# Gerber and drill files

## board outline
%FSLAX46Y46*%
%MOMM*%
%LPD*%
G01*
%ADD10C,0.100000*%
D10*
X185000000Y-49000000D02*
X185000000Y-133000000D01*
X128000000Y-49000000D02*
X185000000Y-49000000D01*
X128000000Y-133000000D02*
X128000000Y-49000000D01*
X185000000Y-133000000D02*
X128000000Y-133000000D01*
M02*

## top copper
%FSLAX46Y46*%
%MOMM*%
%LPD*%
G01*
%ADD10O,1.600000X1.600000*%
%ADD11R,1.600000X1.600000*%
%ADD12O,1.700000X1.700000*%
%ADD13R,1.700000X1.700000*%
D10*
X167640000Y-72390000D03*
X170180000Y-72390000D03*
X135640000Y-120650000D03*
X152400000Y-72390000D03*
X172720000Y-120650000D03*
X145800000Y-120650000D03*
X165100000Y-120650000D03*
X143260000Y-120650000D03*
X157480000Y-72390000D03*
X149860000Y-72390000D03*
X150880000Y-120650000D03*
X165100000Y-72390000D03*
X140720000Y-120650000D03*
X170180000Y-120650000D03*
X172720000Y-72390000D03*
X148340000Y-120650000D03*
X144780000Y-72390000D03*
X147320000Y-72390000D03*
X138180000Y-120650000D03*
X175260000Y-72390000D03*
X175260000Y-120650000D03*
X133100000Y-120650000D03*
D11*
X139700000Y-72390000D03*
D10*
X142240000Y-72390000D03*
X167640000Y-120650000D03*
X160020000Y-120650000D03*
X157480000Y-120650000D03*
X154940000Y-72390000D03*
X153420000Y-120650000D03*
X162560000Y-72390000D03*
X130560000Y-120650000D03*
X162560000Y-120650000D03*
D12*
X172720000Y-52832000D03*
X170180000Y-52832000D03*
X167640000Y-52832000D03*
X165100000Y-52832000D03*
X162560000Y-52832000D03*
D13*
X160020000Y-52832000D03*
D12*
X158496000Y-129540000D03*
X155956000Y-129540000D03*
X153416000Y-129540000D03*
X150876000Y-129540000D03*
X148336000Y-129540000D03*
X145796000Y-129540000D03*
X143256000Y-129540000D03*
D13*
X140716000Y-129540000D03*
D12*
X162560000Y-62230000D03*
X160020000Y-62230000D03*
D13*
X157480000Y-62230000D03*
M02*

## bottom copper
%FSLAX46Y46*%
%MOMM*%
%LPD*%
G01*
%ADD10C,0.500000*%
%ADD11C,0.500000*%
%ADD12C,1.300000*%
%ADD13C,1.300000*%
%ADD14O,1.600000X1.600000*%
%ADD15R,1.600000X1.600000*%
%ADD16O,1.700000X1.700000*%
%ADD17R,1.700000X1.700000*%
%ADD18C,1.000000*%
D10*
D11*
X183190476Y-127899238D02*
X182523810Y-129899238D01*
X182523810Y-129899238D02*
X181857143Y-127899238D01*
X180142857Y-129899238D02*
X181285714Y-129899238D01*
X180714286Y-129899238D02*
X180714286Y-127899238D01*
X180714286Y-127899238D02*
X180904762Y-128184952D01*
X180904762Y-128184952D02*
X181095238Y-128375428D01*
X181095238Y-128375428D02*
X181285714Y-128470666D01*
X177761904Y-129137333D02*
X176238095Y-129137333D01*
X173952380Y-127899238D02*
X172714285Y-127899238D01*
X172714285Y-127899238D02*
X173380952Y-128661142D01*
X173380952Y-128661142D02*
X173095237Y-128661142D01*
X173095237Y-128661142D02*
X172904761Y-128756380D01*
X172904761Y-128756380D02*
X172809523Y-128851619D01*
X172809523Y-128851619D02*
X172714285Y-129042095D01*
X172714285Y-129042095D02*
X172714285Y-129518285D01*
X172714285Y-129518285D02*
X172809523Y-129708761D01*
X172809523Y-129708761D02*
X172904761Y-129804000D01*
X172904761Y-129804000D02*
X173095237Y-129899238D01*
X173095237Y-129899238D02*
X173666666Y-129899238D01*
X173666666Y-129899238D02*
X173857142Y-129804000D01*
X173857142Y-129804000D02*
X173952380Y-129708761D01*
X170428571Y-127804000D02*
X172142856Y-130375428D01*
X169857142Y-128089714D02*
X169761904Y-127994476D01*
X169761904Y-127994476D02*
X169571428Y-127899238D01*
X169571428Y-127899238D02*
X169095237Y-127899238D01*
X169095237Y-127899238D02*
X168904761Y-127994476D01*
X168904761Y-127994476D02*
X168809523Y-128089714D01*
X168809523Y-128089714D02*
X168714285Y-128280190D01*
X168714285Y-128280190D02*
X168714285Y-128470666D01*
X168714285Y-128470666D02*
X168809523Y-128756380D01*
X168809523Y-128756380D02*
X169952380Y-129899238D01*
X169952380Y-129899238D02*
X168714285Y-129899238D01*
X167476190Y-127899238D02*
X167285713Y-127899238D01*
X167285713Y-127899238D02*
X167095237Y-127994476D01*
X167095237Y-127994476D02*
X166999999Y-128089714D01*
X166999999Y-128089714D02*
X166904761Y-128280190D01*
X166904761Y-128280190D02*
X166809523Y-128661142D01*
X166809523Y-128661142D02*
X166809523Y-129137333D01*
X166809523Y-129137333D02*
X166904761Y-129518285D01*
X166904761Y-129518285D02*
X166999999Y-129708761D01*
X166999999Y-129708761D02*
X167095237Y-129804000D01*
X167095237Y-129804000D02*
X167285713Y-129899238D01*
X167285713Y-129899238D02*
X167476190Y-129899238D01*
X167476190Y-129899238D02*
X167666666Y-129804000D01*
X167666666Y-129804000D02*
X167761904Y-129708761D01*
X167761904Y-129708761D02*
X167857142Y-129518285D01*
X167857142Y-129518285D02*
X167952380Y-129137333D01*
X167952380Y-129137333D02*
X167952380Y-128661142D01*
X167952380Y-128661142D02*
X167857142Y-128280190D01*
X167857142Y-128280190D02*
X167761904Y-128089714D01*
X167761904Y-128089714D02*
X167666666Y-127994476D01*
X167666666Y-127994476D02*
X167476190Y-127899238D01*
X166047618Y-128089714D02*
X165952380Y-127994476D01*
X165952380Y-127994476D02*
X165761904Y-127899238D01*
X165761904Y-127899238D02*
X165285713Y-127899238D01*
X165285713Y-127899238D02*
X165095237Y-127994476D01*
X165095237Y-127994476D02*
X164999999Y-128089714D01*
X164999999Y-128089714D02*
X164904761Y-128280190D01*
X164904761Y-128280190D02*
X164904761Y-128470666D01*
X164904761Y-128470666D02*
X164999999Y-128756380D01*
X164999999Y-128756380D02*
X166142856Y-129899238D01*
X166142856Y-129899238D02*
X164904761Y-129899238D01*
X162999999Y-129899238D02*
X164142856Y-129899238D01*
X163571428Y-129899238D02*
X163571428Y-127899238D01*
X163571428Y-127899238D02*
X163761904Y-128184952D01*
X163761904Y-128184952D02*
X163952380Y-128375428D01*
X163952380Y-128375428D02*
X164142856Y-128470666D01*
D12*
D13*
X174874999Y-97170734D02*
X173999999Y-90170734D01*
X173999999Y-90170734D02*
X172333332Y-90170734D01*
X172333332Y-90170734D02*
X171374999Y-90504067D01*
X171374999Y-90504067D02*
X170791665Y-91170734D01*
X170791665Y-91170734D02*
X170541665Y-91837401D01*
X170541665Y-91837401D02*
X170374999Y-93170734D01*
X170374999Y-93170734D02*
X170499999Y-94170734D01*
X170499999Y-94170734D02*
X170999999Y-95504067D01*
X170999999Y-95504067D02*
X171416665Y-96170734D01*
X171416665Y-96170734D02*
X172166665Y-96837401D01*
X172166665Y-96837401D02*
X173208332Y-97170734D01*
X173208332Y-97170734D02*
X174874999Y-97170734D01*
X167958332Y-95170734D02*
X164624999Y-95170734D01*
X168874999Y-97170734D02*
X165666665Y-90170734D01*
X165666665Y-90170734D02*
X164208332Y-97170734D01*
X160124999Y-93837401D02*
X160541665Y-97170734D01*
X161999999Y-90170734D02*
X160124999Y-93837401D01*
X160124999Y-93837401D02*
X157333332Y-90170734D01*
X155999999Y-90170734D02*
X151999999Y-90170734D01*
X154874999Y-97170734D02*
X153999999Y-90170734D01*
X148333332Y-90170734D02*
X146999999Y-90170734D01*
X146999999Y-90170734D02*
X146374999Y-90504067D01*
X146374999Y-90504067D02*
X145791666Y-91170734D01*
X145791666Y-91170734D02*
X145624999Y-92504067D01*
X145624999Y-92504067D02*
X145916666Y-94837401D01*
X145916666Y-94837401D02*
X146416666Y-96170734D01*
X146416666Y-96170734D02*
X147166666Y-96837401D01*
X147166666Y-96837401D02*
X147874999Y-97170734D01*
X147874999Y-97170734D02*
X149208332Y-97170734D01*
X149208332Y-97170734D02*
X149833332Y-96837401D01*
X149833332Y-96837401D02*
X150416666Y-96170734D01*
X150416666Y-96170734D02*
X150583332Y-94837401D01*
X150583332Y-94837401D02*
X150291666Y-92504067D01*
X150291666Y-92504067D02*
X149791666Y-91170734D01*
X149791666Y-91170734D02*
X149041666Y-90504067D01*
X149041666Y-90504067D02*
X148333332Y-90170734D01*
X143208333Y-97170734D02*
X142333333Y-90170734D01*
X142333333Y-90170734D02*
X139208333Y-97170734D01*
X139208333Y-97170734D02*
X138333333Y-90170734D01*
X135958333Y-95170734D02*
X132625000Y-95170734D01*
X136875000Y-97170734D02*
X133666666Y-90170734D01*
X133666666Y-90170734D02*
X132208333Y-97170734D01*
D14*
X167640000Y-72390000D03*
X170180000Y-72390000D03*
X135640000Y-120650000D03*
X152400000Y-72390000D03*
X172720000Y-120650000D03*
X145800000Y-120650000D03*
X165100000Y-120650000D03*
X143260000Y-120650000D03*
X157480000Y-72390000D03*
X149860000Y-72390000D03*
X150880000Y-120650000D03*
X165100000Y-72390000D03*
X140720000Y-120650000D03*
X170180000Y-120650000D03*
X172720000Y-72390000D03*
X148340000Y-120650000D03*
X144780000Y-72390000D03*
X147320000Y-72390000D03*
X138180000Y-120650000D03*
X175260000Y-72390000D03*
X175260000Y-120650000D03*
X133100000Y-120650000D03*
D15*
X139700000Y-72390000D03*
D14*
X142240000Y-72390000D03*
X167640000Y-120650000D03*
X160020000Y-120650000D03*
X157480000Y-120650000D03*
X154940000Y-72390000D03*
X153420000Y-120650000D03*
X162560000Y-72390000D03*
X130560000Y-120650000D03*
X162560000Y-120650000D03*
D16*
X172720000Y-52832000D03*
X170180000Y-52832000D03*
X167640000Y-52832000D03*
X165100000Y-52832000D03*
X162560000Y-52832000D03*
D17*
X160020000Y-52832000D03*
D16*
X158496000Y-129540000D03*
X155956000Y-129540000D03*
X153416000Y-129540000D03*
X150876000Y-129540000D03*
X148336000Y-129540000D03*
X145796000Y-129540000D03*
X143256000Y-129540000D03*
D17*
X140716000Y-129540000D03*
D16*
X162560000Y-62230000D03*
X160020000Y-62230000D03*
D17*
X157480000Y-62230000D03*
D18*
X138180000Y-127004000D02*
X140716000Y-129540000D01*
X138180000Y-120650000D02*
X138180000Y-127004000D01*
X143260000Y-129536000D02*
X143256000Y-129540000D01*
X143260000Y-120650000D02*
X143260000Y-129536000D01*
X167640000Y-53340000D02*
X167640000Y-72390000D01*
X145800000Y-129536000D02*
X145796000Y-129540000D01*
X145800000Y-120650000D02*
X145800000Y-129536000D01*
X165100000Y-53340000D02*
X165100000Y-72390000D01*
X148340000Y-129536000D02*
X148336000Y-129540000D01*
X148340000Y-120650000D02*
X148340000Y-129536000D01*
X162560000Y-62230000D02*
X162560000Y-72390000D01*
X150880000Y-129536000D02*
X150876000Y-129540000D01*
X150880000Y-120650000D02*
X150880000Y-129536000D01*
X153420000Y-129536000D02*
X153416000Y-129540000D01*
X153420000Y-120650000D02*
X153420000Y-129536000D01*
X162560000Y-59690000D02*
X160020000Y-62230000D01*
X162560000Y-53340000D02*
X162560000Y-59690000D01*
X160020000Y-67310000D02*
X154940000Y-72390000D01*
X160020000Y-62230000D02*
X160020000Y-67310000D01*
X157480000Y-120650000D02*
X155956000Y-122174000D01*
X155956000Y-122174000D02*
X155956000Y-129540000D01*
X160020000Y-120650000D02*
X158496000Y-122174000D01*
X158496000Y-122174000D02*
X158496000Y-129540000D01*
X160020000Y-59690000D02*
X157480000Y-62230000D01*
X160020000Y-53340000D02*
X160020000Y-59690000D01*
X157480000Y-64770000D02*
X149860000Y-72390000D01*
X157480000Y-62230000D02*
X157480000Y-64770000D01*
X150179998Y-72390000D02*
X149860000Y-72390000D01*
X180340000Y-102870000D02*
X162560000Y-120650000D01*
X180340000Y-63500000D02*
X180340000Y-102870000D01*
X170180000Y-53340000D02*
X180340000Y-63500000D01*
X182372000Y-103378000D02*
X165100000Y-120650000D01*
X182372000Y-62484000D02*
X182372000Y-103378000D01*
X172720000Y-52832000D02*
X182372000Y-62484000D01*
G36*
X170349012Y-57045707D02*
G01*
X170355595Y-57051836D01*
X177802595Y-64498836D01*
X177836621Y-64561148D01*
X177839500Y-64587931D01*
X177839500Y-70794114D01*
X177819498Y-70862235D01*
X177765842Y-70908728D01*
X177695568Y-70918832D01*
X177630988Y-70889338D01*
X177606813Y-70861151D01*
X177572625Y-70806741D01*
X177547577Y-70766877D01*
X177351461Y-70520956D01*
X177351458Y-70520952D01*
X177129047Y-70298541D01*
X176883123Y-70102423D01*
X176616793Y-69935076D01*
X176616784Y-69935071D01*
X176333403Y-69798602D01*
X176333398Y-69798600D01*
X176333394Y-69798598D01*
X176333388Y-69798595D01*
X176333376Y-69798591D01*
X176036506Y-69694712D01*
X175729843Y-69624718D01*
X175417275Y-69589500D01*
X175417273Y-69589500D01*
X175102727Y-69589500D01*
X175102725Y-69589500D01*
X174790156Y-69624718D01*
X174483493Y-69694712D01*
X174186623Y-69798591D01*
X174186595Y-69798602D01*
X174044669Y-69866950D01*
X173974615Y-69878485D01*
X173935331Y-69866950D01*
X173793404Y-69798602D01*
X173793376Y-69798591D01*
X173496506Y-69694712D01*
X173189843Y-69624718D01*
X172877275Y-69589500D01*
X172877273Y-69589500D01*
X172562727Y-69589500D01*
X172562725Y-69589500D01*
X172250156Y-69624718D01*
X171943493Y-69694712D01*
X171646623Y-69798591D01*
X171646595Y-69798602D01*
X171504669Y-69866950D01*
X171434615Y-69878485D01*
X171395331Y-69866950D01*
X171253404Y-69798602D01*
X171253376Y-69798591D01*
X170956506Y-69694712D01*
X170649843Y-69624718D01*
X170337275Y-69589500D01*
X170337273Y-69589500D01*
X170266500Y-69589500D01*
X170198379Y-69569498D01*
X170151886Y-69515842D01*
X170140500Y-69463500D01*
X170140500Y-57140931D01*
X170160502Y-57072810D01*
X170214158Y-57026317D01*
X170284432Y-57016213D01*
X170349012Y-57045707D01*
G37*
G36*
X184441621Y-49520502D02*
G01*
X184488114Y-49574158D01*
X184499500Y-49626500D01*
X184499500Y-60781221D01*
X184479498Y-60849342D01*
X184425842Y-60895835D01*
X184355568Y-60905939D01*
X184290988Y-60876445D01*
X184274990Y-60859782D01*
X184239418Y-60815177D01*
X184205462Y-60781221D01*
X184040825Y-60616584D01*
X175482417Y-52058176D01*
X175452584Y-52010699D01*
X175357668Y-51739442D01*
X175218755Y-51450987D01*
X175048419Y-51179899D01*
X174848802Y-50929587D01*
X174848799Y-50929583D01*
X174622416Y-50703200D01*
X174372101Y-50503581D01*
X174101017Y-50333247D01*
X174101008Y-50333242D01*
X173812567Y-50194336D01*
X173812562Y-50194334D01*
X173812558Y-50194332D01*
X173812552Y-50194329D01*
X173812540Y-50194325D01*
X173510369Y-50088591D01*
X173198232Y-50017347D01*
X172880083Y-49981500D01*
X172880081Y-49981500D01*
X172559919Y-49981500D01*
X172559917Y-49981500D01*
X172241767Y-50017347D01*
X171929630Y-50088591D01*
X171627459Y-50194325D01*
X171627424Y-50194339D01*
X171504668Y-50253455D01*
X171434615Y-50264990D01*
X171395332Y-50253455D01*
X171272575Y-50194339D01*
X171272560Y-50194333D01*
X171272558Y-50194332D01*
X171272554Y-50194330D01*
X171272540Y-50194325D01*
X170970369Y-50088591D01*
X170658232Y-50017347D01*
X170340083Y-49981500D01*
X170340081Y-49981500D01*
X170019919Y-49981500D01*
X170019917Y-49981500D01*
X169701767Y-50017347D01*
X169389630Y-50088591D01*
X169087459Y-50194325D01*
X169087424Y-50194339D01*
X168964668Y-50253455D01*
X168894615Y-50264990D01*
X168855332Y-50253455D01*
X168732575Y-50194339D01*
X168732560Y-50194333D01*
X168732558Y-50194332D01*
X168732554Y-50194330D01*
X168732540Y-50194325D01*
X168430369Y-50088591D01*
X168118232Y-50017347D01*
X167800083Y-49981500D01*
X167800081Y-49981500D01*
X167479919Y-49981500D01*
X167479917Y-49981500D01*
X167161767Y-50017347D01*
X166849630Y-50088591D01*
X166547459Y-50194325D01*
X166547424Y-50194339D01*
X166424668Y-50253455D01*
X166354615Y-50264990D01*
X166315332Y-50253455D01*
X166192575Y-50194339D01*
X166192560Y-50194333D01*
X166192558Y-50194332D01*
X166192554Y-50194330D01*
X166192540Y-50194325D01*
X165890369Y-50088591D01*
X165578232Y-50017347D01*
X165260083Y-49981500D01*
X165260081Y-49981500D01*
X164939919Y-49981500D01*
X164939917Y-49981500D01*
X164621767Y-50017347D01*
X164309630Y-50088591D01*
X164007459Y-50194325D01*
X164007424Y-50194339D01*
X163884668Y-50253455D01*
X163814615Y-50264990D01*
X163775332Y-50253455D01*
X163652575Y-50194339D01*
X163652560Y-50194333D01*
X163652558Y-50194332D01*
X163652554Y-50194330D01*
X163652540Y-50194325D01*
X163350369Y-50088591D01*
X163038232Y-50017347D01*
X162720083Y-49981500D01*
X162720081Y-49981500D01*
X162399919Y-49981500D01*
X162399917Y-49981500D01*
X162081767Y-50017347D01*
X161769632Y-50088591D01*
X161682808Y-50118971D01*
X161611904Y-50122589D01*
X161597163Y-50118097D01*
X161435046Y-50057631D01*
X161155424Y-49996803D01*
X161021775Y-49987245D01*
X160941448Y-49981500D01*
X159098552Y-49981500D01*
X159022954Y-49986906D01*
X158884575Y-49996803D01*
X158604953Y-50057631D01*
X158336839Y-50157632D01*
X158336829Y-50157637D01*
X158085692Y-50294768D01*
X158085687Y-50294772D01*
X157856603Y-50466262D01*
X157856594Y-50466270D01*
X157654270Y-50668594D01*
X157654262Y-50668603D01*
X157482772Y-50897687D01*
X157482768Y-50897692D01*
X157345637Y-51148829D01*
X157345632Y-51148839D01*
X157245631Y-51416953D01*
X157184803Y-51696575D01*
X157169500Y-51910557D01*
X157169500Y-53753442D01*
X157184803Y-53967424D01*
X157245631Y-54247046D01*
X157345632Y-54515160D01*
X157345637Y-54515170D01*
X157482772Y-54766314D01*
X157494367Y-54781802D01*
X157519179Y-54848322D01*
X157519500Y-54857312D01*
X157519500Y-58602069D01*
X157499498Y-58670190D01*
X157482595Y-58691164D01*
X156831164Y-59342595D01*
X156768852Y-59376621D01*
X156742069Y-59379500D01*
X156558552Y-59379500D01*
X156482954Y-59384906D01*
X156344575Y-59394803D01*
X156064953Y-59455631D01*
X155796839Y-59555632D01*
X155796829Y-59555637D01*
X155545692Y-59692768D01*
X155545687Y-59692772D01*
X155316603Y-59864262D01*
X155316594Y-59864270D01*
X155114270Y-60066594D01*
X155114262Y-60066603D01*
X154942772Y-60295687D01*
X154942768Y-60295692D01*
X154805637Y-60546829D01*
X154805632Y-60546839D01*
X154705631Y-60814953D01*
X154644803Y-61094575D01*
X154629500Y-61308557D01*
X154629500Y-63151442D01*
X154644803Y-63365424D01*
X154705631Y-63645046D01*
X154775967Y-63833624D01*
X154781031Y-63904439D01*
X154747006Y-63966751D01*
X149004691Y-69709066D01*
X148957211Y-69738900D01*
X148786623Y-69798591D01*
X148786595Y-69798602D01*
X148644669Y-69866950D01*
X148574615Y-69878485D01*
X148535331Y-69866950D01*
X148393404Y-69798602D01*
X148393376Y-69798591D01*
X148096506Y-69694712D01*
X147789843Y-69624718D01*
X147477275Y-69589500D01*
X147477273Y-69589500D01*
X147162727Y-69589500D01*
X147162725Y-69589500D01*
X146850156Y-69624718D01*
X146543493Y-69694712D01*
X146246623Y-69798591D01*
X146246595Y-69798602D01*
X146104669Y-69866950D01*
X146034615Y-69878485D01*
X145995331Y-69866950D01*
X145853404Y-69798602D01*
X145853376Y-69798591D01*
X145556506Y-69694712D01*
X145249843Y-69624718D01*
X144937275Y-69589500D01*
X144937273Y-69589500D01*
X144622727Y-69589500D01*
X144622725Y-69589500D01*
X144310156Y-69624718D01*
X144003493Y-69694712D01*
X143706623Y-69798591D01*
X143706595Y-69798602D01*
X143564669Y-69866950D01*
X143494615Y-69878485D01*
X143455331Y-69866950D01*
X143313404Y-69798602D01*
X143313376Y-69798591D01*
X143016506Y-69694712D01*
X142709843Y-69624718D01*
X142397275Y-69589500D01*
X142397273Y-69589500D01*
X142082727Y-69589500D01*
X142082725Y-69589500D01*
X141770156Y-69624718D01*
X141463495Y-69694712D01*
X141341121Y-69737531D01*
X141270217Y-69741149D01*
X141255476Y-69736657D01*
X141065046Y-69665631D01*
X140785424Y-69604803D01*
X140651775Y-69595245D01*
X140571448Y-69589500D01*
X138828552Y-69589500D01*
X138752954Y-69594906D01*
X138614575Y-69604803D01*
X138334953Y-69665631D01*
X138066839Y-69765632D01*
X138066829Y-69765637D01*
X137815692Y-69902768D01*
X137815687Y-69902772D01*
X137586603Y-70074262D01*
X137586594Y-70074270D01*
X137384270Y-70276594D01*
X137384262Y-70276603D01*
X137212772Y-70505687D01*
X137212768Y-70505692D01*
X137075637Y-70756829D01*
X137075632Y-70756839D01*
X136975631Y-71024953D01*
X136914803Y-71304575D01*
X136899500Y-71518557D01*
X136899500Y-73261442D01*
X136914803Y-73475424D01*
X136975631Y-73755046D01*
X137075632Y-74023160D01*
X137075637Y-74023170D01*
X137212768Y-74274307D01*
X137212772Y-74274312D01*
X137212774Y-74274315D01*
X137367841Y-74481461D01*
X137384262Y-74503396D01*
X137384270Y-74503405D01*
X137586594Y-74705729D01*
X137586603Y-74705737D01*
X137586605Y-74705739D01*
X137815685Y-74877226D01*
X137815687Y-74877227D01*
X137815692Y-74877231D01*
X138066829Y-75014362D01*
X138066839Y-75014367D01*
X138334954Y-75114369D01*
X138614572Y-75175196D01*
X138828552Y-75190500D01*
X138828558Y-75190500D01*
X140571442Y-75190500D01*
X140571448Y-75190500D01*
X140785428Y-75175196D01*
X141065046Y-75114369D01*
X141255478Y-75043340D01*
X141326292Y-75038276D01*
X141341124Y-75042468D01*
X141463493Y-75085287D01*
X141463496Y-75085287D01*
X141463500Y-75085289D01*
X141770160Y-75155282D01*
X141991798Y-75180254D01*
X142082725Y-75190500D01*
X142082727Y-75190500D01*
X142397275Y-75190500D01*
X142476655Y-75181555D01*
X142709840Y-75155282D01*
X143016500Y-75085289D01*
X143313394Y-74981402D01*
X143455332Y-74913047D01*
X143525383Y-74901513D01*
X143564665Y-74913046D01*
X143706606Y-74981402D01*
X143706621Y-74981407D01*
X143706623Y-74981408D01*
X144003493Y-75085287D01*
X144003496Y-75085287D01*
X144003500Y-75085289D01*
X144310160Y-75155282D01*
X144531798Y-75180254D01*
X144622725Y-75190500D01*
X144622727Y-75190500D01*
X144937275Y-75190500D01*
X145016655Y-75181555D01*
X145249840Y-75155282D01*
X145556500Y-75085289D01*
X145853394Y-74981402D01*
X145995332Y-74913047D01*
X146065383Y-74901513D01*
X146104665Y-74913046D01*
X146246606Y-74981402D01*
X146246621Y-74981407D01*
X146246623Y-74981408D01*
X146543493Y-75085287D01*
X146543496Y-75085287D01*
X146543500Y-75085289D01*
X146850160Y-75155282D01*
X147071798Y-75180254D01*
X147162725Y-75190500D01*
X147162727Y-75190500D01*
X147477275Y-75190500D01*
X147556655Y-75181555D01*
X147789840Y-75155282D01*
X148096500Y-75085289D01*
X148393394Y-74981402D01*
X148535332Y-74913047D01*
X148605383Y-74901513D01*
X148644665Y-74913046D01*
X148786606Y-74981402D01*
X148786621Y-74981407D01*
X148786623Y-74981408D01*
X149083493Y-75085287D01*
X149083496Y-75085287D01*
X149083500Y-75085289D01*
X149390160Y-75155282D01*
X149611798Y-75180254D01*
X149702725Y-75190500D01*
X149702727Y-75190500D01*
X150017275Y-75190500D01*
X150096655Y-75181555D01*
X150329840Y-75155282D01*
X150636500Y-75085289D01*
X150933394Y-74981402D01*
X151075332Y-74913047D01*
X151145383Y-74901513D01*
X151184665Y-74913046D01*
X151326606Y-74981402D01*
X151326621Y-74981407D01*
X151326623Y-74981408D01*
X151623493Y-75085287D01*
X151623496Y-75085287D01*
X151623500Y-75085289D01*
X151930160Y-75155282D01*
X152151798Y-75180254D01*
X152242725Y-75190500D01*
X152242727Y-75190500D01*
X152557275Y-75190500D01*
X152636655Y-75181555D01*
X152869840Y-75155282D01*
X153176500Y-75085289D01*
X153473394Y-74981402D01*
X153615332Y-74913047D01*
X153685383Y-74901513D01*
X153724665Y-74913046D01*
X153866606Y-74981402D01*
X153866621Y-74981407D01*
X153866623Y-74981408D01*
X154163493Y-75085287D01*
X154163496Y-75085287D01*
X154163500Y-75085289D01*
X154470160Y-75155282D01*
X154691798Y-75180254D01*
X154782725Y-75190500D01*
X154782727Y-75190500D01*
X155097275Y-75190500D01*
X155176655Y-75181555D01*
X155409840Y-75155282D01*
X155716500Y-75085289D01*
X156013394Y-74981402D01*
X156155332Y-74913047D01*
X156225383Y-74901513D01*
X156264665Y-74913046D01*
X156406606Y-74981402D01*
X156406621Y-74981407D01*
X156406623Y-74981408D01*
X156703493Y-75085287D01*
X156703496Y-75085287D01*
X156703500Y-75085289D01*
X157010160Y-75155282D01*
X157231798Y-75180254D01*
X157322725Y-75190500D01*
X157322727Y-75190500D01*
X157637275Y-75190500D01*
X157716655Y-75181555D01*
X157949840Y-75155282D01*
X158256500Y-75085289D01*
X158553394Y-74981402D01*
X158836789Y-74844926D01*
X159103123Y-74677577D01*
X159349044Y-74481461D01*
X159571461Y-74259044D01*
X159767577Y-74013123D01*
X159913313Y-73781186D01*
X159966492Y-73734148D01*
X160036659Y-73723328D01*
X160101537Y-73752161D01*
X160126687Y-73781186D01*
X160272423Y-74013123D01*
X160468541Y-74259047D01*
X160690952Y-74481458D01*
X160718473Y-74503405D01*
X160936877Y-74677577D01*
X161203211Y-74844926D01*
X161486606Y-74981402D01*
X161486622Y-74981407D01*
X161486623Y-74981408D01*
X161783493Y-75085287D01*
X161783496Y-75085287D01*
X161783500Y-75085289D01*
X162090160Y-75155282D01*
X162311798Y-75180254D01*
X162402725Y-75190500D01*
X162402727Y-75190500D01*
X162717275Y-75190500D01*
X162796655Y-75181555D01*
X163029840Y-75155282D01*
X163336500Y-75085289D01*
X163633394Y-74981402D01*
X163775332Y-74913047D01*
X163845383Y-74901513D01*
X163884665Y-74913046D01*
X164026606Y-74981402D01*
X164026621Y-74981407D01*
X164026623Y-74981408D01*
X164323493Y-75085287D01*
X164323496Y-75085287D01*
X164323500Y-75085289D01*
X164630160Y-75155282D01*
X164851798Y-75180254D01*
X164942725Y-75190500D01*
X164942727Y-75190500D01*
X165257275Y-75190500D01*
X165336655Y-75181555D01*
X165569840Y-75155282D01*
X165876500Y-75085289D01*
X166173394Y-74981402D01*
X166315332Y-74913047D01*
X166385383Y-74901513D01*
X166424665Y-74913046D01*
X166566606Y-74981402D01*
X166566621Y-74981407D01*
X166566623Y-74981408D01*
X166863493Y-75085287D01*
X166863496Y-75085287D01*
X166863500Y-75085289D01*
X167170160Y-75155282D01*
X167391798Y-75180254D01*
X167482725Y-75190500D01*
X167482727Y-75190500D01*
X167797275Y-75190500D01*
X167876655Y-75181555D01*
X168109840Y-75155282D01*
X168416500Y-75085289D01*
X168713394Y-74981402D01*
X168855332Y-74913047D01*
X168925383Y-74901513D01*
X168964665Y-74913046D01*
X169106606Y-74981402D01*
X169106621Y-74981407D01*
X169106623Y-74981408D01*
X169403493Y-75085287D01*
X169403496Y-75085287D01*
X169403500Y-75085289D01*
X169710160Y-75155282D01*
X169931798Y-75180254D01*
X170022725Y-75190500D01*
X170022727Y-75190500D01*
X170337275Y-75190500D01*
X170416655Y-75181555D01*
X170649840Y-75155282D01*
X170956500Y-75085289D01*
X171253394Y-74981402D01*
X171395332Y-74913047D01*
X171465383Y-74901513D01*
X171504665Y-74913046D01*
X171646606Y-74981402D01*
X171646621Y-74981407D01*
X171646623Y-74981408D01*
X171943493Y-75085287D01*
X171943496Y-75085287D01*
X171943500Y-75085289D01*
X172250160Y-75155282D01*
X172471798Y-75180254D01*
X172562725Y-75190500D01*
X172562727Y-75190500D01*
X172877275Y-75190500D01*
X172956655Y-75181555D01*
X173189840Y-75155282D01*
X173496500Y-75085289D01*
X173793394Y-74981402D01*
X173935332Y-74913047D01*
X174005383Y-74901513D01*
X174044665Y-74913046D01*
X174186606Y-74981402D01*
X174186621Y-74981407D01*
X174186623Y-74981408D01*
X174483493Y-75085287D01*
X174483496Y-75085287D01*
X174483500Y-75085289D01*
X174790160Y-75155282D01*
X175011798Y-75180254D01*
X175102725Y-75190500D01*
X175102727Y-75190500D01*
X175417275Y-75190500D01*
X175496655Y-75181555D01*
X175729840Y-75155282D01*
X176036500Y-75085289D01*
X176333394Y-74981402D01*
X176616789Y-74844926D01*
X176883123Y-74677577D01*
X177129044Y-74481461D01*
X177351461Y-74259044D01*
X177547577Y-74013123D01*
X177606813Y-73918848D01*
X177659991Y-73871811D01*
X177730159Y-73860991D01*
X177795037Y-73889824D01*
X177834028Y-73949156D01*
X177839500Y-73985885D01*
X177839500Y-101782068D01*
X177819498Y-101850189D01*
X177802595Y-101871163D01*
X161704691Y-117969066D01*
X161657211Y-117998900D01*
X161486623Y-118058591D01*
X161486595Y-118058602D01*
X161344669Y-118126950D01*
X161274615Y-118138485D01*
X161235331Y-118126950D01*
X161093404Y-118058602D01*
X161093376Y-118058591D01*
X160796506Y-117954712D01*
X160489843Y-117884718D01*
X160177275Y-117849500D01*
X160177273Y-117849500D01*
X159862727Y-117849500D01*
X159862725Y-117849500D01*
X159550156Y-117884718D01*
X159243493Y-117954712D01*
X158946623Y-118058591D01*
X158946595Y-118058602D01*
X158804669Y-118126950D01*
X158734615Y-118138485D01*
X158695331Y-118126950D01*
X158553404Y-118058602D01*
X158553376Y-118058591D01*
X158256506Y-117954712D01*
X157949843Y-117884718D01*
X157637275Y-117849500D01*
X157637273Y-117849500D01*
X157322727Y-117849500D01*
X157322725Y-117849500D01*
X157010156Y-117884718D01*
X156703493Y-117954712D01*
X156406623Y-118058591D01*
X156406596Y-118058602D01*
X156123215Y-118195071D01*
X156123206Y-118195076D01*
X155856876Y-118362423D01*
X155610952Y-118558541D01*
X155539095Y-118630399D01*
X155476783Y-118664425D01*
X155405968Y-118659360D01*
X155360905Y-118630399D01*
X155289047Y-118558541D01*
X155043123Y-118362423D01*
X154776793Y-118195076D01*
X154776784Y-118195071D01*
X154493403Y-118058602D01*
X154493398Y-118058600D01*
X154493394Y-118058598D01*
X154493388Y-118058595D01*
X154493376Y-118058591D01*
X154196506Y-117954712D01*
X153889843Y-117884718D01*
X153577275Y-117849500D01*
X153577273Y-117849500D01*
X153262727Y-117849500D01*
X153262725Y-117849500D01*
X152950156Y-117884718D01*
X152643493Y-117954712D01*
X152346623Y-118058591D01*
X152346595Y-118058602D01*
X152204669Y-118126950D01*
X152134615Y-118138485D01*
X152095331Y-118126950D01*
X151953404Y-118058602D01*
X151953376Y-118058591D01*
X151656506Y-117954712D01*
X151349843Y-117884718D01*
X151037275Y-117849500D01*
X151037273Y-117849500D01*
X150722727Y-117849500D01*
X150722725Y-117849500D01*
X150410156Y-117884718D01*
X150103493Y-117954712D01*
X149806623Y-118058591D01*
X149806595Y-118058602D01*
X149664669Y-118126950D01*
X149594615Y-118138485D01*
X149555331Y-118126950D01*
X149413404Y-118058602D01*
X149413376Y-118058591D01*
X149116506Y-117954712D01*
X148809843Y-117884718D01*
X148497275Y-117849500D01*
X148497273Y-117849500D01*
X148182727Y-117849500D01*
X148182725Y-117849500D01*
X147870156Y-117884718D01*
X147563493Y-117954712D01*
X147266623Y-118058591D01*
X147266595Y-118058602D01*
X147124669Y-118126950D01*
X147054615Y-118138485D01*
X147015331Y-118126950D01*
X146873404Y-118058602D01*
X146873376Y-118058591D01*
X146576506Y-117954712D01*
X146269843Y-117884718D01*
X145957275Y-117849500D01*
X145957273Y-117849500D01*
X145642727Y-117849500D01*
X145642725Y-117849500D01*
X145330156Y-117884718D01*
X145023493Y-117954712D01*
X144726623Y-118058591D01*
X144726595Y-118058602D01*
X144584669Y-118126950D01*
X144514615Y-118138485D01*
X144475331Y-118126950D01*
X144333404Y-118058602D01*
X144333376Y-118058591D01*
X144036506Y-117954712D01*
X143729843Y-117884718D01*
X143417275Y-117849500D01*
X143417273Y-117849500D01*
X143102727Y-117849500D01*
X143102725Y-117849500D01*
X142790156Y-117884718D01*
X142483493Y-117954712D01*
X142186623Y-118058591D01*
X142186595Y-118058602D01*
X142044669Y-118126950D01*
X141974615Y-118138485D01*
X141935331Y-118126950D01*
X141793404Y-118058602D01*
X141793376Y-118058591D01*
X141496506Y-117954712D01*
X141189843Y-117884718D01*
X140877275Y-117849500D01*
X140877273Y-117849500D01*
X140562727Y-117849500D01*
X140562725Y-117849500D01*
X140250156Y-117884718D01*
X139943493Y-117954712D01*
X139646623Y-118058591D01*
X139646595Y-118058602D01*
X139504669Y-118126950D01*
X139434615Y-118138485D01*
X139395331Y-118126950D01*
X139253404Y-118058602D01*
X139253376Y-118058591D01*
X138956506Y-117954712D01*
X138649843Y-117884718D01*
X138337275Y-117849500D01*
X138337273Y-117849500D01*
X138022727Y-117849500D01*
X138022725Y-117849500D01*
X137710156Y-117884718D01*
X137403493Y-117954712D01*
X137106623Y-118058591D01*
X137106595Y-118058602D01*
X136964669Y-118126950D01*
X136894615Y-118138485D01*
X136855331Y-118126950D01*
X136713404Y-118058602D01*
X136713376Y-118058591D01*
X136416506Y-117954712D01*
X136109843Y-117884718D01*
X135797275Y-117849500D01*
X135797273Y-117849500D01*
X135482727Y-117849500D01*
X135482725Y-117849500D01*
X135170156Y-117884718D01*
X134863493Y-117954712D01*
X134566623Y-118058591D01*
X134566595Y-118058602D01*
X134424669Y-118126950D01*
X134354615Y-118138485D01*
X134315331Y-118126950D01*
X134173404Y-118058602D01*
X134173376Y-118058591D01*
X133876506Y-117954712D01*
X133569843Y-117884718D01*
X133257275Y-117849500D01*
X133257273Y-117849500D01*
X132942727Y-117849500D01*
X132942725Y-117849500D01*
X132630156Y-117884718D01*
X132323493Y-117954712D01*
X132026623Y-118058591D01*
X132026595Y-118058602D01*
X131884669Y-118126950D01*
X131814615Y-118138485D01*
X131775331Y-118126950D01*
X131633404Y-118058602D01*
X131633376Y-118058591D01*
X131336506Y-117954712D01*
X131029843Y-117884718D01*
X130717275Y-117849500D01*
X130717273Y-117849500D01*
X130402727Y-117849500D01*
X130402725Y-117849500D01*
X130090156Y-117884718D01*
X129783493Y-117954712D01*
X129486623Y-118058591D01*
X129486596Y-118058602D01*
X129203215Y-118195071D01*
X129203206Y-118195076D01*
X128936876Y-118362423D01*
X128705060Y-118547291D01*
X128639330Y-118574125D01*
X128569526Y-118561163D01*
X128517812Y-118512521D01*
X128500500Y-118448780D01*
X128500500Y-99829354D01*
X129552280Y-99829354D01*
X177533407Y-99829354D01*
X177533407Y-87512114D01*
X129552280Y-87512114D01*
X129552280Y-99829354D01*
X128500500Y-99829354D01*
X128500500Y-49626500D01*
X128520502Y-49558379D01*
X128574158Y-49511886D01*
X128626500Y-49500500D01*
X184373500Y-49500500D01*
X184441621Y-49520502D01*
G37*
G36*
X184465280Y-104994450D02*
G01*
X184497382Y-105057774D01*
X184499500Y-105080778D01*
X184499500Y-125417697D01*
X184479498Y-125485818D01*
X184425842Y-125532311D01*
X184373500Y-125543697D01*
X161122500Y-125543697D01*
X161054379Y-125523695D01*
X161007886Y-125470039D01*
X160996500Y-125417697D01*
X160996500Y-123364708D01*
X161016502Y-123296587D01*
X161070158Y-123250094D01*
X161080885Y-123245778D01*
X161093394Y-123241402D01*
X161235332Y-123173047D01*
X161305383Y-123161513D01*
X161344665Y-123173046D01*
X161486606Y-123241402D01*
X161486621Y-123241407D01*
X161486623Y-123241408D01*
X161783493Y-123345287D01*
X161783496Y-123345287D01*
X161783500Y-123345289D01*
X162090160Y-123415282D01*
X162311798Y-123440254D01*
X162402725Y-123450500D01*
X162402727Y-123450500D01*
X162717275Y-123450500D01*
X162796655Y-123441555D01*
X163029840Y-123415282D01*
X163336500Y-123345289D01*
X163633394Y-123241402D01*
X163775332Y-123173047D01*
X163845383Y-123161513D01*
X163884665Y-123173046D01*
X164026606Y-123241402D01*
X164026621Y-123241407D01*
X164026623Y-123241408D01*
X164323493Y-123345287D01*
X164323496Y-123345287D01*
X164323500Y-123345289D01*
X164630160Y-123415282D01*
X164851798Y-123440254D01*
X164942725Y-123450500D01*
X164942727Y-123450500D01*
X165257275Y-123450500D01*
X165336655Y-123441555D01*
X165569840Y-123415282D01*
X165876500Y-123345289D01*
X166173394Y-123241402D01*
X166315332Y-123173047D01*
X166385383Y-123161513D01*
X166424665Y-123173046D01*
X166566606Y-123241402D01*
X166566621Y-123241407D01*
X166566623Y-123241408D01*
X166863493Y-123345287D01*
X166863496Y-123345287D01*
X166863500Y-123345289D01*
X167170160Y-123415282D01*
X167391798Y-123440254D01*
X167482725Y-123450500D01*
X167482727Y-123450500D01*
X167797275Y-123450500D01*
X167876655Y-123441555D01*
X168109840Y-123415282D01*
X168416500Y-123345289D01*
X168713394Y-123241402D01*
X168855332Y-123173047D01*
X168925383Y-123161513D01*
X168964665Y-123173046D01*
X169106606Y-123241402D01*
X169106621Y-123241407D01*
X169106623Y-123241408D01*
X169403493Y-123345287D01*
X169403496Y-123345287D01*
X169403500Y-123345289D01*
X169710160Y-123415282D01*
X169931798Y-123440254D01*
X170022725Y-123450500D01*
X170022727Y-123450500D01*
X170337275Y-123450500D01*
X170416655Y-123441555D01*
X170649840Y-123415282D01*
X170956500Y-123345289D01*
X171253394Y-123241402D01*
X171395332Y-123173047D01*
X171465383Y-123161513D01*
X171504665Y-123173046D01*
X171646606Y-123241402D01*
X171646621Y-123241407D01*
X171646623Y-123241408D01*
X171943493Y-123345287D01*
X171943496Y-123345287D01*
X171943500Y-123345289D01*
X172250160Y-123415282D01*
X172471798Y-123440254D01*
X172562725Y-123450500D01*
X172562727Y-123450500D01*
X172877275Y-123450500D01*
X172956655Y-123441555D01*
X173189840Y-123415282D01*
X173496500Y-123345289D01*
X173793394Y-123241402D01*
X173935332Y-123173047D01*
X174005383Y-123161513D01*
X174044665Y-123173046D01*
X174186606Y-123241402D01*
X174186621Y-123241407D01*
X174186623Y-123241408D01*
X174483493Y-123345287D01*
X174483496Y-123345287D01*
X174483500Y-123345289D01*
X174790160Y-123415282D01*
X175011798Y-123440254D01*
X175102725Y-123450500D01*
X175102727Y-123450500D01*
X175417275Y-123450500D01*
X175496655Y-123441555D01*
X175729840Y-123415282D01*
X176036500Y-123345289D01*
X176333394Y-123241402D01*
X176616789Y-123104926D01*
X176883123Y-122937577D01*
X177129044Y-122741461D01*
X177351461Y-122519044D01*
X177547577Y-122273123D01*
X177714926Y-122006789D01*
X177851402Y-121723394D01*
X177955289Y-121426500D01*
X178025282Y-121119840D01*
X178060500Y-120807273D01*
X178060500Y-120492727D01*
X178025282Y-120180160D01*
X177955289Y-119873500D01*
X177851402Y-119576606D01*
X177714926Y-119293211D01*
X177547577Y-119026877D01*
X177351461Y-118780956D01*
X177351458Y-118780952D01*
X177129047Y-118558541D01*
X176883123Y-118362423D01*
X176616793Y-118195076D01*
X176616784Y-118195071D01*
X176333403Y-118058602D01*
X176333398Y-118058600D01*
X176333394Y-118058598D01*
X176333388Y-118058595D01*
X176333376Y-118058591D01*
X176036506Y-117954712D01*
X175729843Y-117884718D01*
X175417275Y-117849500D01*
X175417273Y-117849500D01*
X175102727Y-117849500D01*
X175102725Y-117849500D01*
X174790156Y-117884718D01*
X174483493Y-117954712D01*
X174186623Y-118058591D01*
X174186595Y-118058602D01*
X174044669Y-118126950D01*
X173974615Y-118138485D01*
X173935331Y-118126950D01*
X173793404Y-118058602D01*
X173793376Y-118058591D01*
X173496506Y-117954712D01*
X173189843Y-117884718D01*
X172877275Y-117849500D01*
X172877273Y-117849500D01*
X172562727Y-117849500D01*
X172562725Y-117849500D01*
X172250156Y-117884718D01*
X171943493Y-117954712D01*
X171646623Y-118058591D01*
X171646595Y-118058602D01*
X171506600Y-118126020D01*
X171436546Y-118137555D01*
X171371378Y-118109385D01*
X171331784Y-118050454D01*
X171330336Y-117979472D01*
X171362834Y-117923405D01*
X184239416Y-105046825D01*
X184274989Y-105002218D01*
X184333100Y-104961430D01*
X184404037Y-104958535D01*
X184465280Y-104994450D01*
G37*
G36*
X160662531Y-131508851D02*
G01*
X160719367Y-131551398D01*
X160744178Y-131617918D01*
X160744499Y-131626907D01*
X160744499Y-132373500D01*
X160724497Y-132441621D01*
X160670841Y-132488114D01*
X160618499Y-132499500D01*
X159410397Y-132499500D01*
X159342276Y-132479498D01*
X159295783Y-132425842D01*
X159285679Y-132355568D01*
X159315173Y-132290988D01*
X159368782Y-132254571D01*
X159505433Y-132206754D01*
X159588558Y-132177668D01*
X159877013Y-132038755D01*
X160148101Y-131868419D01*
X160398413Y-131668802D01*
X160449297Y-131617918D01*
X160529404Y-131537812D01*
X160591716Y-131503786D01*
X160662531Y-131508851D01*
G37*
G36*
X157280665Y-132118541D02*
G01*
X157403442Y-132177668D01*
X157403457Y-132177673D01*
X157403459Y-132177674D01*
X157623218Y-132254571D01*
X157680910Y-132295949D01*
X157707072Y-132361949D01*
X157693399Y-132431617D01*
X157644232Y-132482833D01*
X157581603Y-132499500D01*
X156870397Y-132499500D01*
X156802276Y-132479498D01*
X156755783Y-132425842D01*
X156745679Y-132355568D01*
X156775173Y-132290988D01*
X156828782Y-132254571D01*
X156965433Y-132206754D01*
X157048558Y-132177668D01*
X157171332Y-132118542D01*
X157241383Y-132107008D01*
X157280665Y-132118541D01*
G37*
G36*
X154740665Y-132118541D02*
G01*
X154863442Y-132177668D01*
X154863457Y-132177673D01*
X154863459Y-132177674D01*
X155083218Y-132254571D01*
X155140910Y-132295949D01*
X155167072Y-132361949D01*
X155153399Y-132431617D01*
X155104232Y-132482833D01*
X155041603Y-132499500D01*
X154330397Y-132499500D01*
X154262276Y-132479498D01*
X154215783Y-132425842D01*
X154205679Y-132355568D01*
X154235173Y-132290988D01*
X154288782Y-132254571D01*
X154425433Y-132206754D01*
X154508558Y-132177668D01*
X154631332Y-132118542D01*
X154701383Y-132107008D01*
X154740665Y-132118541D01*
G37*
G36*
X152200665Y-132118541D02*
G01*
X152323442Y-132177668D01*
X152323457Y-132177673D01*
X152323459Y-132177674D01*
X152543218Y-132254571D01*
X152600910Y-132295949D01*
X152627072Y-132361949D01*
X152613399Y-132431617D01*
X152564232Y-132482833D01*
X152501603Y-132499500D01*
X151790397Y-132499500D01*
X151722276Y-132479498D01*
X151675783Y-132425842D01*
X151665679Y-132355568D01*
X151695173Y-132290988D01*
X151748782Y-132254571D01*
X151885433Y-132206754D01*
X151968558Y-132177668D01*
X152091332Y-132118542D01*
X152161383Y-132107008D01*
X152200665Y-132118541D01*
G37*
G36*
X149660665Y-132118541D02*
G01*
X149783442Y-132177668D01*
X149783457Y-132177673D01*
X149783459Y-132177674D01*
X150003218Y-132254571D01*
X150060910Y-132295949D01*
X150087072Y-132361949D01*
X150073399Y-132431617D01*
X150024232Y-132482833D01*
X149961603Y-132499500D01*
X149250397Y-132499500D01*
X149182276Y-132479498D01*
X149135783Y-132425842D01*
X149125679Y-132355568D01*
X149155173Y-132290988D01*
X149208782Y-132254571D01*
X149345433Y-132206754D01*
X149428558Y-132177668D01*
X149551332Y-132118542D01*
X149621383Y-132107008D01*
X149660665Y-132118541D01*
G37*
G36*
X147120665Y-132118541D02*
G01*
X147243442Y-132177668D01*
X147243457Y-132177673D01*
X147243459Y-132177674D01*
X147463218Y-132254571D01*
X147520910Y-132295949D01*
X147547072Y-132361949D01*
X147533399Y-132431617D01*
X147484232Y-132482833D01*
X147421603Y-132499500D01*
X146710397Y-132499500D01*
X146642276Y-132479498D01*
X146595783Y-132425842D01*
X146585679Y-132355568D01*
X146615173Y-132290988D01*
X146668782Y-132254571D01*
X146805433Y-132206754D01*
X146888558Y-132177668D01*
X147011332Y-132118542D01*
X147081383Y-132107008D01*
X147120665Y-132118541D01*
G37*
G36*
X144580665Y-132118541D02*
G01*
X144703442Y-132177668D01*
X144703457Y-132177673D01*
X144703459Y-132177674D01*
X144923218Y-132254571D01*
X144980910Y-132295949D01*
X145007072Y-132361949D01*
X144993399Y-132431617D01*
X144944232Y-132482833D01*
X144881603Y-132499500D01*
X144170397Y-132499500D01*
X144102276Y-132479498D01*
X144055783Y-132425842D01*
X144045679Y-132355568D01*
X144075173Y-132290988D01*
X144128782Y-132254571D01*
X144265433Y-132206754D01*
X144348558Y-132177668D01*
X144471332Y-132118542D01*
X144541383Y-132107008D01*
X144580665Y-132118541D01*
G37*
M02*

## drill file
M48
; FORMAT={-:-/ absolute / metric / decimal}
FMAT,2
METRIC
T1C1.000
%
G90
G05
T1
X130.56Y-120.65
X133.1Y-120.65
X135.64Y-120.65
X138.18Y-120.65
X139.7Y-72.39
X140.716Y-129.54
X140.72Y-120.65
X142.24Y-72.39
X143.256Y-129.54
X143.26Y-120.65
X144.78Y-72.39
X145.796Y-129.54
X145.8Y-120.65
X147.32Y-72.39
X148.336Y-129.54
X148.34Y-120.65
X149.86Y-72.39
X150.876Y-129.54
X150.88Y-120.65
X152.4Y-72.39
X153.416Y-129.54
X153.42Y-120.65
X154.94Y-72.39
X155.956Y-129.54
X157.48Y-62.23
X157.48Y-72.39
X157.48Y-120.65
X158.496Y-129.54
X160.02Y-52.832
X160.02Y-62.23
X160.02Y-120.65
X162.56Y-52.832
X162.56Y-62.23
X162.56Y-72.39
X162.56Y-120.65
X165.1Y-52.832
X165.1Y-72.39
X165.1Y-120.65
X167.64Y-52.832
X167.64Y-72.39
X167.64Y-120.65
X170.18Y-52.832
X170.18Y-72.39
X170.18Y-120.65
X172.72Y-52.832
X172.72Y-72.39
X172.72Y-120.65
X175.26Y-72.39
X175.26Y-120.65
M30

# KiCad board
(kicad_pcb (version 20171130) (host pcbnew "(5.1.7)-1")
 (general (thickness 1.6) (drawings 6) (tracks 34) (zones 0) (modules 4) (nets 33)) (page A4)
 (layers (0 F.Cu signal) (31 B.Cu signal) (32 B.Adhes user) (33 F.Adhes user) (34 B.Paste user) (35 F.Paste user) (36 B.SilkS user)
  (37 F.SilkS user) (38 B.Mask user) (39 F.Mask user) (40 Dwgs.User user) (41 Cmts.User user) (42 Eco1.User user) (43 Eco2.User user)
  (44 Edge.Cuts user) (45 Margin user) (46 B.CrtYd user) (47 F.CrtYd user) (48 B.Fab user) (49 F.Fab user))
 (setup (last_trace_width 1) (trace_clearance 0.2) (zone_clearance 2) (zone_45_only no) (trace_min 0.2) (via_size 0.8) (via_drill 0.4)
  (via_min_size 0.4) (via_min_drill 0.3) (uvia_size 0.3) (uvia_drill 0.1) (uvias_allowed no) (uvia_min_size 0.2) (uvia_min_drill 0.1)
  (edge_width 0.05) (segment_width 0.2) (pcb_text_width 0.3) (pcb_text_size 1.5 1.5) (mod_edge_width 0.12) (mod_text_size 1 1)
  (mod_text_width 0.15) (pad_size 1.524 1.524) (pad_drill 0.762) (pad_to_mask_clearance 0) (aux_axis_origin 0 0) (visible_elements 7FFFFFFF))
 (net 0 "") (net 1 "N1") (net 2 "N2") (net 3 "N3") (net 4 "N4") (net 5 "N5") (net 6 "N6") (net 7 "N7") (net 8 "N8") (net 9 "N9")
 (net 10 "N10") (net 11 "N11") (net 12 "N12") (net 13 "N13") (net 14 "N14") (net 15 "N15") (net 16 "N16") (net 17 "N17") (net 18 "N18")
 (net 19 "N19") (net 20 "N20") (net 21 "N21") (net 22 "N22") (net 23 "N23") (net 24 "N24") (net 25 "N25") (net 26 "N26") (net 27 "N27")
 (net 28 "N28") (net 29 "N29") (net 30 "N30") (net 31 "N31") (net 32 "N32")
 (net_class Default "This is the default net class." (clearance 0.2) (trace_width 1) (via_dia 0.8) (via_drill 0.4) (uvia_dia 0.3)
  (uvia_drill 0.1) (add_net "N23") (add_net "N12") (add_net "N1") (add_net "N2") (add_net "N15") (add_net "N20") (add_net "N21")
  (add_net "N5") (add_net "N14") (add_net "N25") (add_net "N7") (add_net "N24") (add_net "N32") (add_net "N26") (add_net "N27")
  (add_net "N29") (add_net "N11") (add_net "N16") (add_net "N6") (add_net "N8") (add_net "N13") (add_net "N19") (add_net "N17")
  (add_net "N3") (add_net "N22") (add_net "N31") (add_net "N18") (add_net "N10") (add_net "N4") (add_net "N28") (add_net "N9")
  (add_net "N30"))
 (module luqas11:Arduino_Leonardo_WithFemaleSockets (layer F.Cu) (at 149.86 97.79)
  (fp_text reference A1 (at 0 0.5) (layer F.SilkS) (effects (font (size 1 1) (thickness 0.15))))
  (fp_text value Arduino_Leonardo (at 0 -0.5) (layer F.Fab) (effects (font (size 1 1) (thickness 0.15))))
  (pad 11 thru_hole oval (at 17.78 -25.4 90) (size 1.6 1.6) (drill 1) (layers *.Cu *.Mask) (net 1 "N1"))
  (pad 12 thru_hole oval (at 20.32 -25.4 90) (size 1.6 1.6) (drill 1) (layers *.Cu *.Mask) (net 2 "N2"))
  (pad 30 thru_hole oval (at -14.22 22.86 90) (size 1.6 1.6) (drill 1) (layers *.Cu *.Mask) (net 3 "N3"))
  (pad 6 thru_hole oval (at 2.54 -25.4 90) (size 1.6 1.6) (drill 1) (layers *.Cu *.Mask) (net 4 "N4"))
  (pad 16 thru_hole oval (at 22.86 22.86 90) (size 1.6 1.6) (drill 1) (layers *.Cu *.Mask) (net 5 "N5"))
  (pad 26 thru_hole oval (at -4.06 22.86 90) (size 1.6 1.6) (drill 1) (layers *.Cu *.Mask) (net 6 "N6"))
  (pad 19 thru_hole oval (at 15.24 22.86 90) (size 1.6 1.6) (drill 1) (layers *.Cu *.Mask) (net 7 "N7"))
  (pad 27 thru_hole oval (at -6.6 22.86 90) (size 1.6 1.6) (drill 1) (layers *.Cu *.Mask) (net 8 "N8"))
  (pad 8 thru_hole oval (at 7.62 -25.4 90) (size 1.6 1.6) (drill 1) (layers *.Cu *.Mask) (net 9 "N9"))
  (pad 5 thru_hole oval (at 0 -25.4 90) (size 1.6 1.6) (drill 1) (layers *.Cu *.Mask) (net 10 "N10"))
  (pad 24 thru_hole oval (at 1.02 22.86 90) (size 1.6 1.6) (drill 1) (layers *.Cu *.Mask) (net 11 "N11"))
  (pad 10 thru_hole oval (at 15.24 -25.4 90) (size 1.6 1.6) (drill 1) (layers *.Cu *.Mask) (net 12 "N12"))
  (pad 28 thru_hole oval (at -9.14 22.86 90) (size 1.6 1.6) (drill 1) (layers *.Cu *.Mask) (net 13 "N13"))
  (pad 17 thru_hole oval (at 20.32 22.86 90) (size 1.6 1.6) (drill 1) (layers *.Cu *.Mask) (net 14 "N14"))
  (pad 13 thru_hole oval (at 22.86 -25.4 90) (size 1.6 1.6) (drill 1) (layers *.Cu *.Mask) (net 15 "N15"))
  (pad 25 thru_hole oval (at -1.52 22.86 90) (size 1.6 1.6) (drill 1) (layers *.Cu *.Mask) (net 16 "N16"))
  (pad 3 thru_hole oval (at -5.08 -25.4 90) (size 1.6 1.6) (drill 1) (layers *.Cu *.Mask) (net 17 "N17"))
  (pad 4 thru_hole oval (at -2.54 -25.4 90) (size 1.6 1.6) (drill 1) (layers *.Cu *.Mask) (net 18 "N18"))
  (pad 29 thru_hole oval (at -11.68 22.86 90) (size 1.6 1.6) (drill 1) (layers *.Cu *.Mask) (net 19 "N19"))
  (pad 14 thru_hole oval (at 25.4 -25.4 90) (size 1.6 1.6) (drill 1) (layers *.Cu *.Mask) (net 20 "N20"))
  (pad 15 thru_hole oval (at 25.4 22.86 90) (size 1.6 1.6) (drill 1) (layers *.Cu *.Mask) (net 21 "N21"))
  (pad 31 thru_hole oval (at -16.76 22.86 90) (size 1.6 1.6) (drill 1) (layers *.Cu *.Mask) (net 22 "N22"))
  (pad 1 thru_hole rect (at -10.16 -25.4 90) (size 1.6 1.6) (drill 1) (layers *.Cu *.Mask) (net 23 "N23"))
  (pad 2 thru_hole oval (at -7.62 -25.4 90) (size 1.6 1.6) (drill 1) (layers *.Cu *.Mask) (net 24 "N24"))
  (pad 18 thru_hole oval (at 17.78 22.86 90) (size 1.6 1.6) (drill 1) (layers *.Cu *.Mask) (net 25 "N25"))
  (pad 21 thru_hole oval (at 10.16 22.86 90) (size 1.6 1.6) (drill 1) (layers *.Cu *.Mask) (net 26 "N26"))
  (pad 22 thru_hole oval (at 7.62 22.86 90) (size 1.6 1.6) (drill 1) (layers *.Cu *.Mask) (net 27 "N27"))
  (pad 7 thru_hole oval (at 5.08 -25.4 90) (size 1.6 1.6) (drill 1) (layers *.Cu *.Mask) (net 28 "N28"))
  (pad 23 thru_hole oval (at 3.56 22.86 90) (size 1.6 1.6) (drill 1) (layers *.Cu *.Mask) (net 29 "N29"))
  (pad 9 thru_hole oval (at 12.7 -25.4 90) (size 1.6 1.6) (drill 1) (layers *.Cu *.Mask) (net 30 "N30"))
  (pad 32 thru_hole oval (at -19.3 22.86 90) (size 1.6 1.6) (drill 1) (layers *.Cu *.Mask) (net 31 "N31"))
  (pad 20 thru_hole oval (at 12.7 22.86 90) (size 1.6 1.6) (drill 1) (layers *.Cu *.Mask) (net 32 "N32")))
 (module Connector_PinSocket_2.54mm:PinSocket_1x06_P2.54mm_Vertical (layer F.Cu) (at 160.02 52.832 90)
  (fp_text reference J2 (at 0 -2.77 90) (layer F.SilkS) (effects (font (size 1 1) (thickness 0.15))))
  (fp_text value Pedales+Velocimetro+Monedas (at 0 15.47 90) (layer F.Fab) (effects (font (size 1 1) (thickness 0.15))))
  (pad 6 thru_hole oval (at 0 12.7 90) (size 1.7 1.7) (drill 1) (layers *.Cu *.Mask) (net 7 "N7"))
  (pad 5 thru_hole oval (at 0 10.16 90) (size 1.7 1.7) (drill 1) (layers *.Cu *.Mask) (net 32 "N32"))
  (pad 4 thru_hole oval (at 0 7.62 90) (size 1.7 1.7) (drill 1) (layers *.Cu *.Mask) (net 1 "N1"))
  (pad 3 thru_hole oval (at 0 5.08 90) (size 1.7 1.7) (drill 1) (layers *.Cu *.Mask) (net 12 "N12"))
  (pad 2 thru_hole oval (at 0 2.54 90) (size 1.7 1.7) (drill 1) (layers *.Cu *.Mask) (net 28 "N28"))
  (pad 1 thru_hole rect (at 0 0 90) (size 1.7 1.7) (drill 1) (layers *.Cu *.Mask) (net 10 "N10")))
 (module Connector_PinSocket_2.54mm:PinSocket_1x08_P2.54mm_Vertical (layer F.Cu) (at 140.716 129.54 90)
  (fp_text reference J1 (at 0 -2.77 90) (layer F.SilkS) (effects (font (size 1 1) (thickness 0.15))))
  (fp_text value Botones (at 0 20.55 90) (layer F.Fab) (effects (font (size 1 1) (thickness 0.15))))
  (pad 8 thru_hole oval (at 0 17.78 90) (size 1.7 1.7) (drill 1) (layers *.Cu *.Mask) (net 26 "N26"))
  (pad 7 thru_hole oval (at 0 15.24 90) (size 1.7 1.7) (drill 1) (layers *.Cu *.Mask) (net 27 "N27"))
  (pad 6 thru_hole oval (at 0 12.7 90) (size 1.7 1.7) (drill 1) (layers *.Cu *.Mask) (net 29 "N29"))
  (pad 5 thru_hole oval (at 0 10.16 90) (size 1.7 1.7) (drill 1) (layers *.Cu *.Mask) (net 11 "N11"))
  (pad 4 thru_hole oval (at 0 7.62 90) (size 1.7 1.7) (drill 1) (layers *.Cu *.Mask) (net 16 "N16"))
  (pad 3 thru_hole oval (at 0 5.08 90) (size 1.7 1.7) (drill 1) (layers *.Cu *.Mask) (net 6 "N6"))
  (pad 2 thru_hole oval (at 0 2.54 90) (size 1.7 1.7) (drill 1) (layers *.Cu *.Mask) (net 8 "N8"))
  (pad 1 thru_hole rect (at 0 0 90) (size 1.7 1.7) (drill 1) (layers *.Cu *.Mask) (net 19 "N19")))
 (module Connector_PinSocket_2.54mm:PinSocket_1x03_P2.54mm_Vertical (layer F.Cu) (at 157.48 62.23 90)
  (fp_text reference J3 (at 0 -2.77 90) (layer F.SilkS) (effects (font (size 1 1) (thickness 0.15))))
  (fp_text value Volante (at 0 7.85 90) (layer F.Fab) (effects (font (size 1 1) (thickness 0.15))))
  (pad 3 thru_hole oval (at 0 5.08 90) (size 1.7 1.7) (drill 1) (layers *.Cu *.Mask) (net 30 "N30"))
  (pad 2 thru_hole oval (at 0 2.54 90) (size 1.7 1.7) (drill 1) (layers *.Cu *.Mask) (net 28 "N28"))
  (pad 1 thru_hole rect (at 0 0 90) (size 1.7 1.7) (drill 1) (layers *.Cu *.Mask) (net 10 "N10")))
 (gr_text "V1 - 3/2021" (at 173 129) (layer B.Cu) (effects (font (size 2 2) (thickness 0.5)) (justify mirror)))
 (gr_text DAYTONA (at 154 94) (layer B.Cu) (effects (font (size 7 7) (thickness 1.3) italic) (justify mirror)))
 (gr_line (start 185 49) (end 185 133) (layer Edge.Cuts) (width 0.1))
 (gr_line (start 128 49) (end 185 49) (layer Edge.Cuts) (width 0.1))
 (gr_line (start 128 133) (end 128 49) (layer Edge.Cuts) (width 0.1))
 (gr_line (start 185 133) (end 128 133) (layer Edge.Cuts) (width 0.1))
 (segment (start 138.18 127.004) (end 140.716 129.54) (width 1) (layer B.Cu) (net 19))
 (segment (start 138.18 120.65) (end 138.18 127.004) (width 1) (layer B.Cu) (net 19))
 (segment (start 143.26 129.536) (end 143.256 129.54) (width 1) (layer B.Cu) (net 8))
 (segment (start 143.26 120.65) (end 143.26 129.536) (width 1) (layer B.Cu) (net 8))
 (segment (start 167.64 53.34) (end 167.64 72.39) (width 1) (layer B.Cu) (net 1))
 (segment (start 145.8 129.536) (end 145.796 129.54) (width 1) (layer B.Cu) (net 6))
 (segment (start 145.8 120.65) (end 145.8 129.536) (width 1) (layer B.Cu) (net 6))
 (segment (start 165.1 53.34) (end 165.1 72.39) (width 1) (layer B.Cu) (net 12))
 (segment (start 148.34 129.536) (end 148.336 129.54) (width 1) (layer B.Cu) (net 16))
 (segment (start 148.34 120.65) (end 148.34 129.536) (width 1) (layer B.Cu) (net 16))
 (segment (start 162.56 62.23) (end 162.56 72.39) (width 1) (layer B.Cu) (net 30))
 (segment (start 150.88 129.536) (end 150.876 129.54) (width 1) (layer B.Cu) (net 11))
 (segment (start 150.88 120.65) (end 150.88 129.536) (width 1) (layer B.Cu) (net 11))
 (segment (start 153.42 129.536) (end 153.416 129.54) (width 1) (layer B.Cu) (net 29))
 (segment (start 153.42 120.65) (end 153.42 129.536) (width 1) (layer B.Cu) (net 29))
 (segment (start 162.56 59.69) (end 160.02 62.23) (width 1) (layer B.Cu) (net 28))
 (segment (start 162.56 53.34) (end 162.56 59.69) (width 1) (layer B.Cu) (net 28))
 (segment (start 160.02 67.31) (end 154.94 72.39) (width 1) (layer B.Cu) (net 28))
 (segment (start 160.02 62.23) (end 160.02 67.31) (width 1) (layer B.Cu) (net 28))
 (segment (start 157.48 120.65) (end 155.956 122.174) (width 1) (layer B.Cu) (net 27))
 (segment (start 155.956 122.174) (end 155.956 129.54) (width 1) (layer B.Cu) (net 27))
 (segment (start 160.02 120.65) (end 158.496 122.174) (width 1) (layer B.Cu) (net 26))
 (segment (start 158.496 122.174) (end 158.496 129.54) (width 1) (layer B.Cu) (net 26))
 (segment (start 160.02 59.69) (end 157.48 62.23) (width 1) (layer B.Cu) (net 10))
 (segment (start 160.02 53.34) (end 160.02 59.69) (width 1) (layer B.Cu) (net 10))
 (segment (start 157.48 64.77) (end 149.86 72.39) (width 1) (layer B.Cu) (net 10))
 (segment (start 157.48 62.23) (end 157.48 64.77) (width 1) (layer B.Cu) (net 10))
 (segment (start 150.179998 72.39) (end 149.86 72.39) (width 1) (layer B.Cu) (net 10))
 (segment (start 180.34 102.87) (end 162.56 120.65) (width 1) (layer B.Cu) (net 32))
 (segment (start 180.34 63.5) (end 180.34 102.87) (width 1) (layer B.Cu) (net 32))
 (segment (start 170.18 53.34) (end 180.34 63.5) (width 1) (layer B.Cu) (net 32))
 (segment (start 182.372 103.378) (end 165.1 120.65) (width 1) (layer B.Cu) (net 7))
 (segment (start 182.372 62.484) (end 182.372 103.378) (width 1) (layer B.Cu) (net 7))
 (segment (start 172.72 52.832) (end 182.372 62.484) (width 1) (layer B.Cu) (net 7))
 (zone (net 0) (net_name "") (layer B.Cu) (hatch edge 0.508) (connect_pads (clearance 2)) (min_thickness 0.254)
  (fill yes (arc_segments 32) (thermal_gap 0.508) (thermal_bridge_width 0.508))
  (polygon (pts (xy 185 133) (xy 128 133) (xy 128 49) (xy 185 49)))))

